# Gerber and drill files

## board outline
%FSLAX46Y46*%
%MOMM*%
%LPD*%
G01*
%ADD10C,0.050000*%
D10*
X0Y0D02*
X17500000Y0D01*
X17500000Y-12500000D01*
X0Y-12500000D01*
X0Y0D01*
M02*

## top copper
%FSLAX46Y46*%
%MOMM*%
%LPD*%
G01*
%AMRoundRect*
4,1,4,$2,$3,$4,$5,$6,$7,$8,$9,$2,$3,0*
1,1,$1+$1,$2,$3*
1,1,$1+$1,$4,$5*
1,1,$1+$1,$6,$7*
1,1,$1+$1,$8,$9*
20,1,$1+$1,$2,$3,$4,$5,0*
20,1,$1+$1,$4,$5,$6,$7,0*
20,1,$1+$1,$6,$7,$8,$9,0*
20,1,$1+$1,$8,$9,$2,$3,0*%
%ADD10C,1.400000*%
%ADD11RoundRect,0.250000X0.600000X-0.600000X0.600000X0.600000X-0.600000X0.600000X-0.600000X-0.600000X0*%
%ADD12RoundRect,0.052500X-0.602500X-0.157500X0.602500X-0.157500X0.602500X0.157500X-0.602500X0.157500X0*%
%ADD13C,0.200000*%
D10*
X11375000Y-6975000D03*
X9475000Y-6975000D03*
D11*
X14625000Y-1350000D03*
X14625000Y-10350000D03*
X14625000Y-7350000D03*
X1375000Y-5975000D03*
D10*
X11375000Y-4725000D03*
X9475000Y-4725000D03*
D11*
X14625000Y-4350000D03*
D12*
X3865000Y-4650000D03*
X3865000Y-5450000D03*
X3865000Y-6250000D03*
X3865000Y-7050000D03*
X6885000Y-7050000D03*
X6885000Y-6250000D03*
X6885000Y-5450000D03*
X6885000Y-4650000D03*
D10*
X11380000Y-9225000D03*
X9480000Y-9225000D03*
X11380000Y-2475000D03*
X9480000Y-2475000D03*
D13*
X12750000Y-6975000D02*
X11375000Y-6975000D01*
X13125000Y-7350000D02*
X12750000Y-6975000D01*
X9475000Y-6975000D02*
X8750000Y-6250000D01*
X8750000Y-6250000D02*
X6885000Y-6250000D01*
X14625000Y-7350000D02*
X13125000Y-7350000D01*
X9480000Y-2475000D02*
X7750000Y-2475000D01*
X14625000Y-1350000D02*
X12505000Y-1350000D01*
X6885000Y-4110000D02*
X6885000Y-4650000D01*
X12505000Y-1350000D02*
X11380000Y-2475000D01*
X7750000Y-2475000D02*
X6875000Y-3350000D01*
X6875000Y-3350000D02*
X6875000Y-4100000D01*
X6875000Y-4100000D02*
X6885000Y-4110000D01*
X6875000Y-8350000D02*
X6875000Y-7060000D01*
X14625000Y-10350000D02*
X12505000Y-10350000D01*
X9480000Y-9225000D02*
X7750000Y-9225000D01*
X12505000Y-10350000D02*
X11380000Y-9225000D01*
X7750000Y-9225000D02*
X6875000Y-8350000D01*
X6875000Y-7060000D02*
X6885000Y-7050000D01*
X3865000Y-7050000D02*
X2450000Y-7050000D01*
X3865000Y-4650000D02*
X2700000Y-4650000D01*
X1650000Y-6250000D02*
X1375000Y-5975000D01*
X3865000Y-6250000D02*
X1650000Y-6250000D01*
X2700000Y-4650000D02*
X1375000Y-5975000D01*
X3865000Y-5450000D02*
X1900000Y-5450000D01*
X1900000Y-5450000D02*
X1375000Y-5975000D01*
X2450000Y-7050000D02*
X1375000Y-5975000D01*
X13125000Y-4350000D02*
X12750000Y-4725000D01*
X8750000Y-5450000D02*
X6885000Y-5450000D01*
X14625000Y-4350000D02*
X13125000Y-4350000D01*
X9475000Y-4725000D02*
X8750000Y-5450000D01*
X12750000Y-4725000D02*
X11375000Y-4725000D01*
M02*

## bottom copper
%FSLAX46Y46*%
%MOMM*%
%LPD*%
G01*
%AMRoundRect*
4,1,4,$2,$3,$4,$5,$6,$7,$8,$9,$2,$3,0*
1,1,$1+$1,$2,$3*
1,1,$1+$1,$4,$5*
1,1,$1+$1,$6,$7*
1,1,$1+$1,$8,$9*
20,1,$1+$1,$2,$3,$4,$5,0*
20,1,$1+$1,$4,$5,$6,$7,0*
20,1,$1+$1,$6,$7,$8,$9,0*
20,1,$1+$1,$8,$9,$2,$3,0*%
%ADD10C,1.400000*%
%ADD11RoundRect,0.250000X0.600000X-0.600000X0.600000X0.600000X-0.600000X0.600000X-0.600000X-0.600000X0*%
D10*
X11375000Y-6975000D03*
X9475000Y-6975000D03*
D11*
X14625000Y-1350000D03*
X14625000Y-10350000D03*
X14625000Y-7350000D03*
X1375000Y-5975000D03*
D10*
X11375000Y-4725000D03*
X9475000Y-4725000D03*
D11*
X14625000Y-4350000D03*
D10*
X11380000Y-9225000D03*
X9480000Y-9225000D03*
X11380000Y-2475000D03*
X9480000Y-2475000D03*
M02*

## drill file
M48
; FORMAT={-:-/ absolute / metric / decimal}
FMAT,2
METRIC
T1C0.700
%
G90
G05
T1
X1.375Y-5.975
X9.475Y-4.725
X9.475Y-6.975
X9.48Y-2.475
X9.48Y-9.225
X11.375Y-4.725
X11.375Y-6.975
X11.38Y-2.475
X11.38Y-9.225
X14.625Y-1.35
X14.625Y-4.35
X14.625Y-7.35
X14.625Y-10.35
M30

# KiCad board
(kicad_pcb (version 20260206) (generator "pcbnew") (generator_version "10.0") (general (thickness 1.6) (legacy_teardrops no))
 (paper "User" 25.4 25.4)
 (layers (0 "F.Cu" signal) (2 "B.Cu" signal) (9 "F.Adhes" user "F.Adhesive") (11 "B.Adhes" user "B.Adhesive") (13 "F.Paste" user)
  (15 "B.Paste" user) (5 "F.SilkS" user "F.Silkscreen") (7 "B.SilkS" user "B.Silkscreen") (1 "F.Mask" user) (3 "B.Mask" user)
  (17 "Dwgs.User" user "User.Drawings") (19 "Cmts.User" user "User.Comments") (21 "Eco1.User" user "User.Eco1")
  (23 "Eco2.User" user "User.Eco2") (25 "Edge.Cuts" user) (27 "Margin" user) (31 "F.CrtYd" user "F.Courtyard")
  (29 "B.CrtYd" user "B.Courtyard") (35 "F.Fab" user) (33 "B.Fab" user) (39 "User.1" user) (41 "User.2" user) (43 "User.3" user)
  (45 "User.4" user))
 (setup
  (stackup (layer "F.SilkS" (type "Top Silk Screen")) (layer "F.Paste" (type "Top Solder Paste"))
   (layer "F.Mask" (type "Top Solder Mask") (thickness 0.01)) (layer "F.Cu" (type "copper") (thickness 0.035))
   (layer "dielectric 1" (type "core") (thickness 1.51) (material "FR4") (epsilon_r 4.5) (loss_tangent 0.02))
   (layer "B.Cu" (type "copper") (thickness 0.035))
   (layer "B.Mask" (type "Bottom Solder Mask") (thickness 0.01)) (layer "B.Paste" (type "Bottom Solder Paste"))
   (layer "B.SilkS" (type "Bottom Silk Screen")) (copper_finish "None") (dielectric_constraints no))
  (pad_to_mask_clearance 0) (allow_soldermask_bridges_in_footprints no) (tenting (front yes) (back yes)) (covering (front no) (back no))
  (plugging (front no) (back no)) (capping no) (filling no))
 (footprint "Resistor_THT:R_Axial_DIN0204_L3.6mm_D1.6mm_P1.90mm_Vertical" (layer "F.Cu") (at 11.375 6.975 180)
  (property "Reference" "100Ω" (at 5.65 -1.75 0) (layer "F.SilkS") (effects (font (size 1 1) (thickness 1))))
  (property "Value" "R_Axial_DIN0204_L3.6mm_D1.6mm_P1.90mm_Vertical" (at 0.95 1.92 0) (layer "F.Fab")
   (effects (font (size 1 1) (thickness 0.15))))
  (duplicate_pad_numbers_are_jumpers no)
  (pad "1" thru_hole circle (at 0 0 180) (size 1.4 1.4) (drill 0.7) (layers "*.Cu" "*.Mask") (remove_unused_layers no) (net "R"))
  (pad "2" thru_hole circle (at 1.9 0 180) (size 1.4 1.4) (drill 0.7) (layers "*.Cu" "*.Mask") (remove_unused_layers no) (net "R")))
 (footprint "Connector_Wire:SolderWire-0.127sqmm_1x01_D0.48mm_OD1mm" (layer "F.Cu") (at 14.625 1.35 90)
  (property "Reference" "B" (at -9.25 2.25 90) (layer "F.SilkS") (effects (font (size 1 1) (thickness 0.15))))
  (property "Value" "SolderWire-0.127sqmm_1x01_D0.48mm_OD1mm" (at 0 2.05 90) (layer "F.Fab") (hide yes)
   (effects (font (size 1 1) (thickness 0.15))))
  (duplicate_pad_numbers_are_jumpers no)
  (pad "1" thru_hole roundrect (at 0 0 90) (size 1.7 1.7) (drill 0.7) (layers "*.Cu" "*.Mask") (remove_unused_layers no)
   (roundrect_rratio 0.147059) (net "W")))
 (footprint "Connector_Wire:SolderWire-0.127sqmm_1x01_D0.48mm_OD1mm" (layer "F.Cu") (at 14.625 10.35 90)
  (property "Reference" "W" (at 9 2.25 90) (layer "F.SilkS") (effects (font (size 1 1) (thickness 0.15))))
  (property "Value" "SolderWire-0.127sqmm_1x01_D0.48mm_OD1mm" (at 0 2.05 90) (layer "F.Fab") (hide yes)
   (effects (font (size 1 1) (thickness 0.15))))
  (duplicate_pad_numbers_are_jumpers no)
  (pad "1" thru_hole roundrect (at 0 0 90) (size 1.7 1.7) (drill 0.7) (layers "*.Cu" "*.Mask") (remove_unused_layers no)
   (roundrect_rratio 0.147059) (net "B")))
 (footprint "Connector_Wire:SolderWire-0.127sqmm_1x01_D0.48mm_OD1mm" (layer "F.Cu") (at 14.625 7.35 90)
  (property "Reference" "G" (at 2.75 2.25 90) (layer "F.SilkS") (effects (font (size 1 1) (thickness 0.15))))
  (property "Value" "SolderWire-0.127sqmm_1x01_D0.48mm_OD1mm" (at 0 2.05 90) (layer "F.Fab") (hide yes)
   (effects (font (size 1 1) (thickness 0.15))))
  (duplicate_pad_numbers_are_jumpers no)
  (pad "1" thru_hole roundrect (at 0 0 90) (size 1.7 1.7) (drill 0.7) (layers "*.Cu" "*.Mask") (remove_unused_layers no)
   (roundrect_rratio 0.147059) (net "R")))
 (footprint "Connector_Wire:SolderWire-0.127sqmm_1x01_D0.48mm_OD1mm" (layer "F.Cu") (at 1.375 5.975 90)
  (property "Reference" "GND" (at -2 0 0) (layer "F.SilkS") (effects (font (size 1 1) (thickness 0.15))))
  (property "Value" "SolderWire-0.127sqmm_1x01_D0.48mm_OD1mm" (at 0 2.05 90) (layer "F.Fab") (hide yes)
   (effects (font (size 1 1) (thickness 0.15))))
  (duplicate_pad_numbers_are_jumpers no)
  (pad "1" thru_hole roundrect (at 0 0 90) (size 1.7 1.7) (drill 0.7) (layers "*.Cu" "*.Mask") (remove_unused_layers no)
   (roundrect_rratio 0.147059) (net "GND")))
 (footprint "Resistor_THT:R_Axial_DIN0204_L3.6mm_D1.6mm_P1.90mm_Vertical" (layer "F.Cu") (at 11.375 4.725 180)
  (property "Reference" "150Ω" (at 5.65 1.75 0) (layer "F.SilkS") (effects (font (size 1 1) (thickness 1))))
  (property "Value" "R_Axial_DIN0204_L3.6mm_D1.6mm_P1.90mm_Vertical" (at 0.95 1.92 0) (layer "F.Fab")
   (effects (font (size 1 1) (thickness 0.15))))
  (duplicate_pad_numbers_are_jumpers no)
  (pad "1" thru_hole circle (at 0 0 180) (size 1.4 1.4) (drill 0.7) (layers "*.Cu" "*.Mask") (remove_unused_layers no) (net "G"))
  (pad "2" thru_hole circle (at 1.9 0 180) (size 1.4 1.4) (drill 0.7) (layers "*.Cu" "*.Mask") (remove_unused_layers no) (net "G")))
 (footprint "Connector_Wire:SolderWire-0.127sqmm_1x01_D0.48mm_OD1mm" (layer "F.Cu") (at 14.625 4.35 90)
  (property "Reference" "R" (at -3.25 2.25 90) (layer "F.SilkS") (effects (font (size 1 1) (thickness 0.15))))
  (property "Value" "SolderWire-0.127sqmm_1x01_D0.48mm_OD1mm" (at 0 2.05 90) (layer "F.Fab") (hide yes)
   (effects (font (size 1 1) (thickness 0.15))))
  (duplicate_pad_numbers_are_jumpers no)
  (pad "1" thru_hole roundrect (at 0 0 90) (size 1.7 1.7) (drill 0.7) (layers "*.Cu" "*.Mask") (remove_unused_layers no)
   (roundrect_rratio 0.147059) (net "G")))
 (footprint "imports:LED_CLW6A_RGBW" (layer "F.Cu") (at 5.375 5.85)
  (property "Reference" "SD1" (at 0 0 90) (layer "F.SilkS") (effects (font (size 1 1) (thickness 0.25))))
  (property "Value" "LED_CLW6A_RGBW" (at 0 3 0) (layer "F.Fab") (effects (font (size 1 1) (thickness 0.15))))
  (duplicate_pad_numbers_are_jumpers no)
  (pad "1" smd roundrect (at -1.51 -1.2) (size 1.31 0.42) (layers "F.Cu" "F.Mask" "F.Paste") (roundrect_rratio 0.125) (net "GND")
   (solder_mask_margin 0.102))
  (pad "2" smd roundrect (at -1.51 -0.4) (size 1.31 0.42) (layers "F.Cu" "F.Mask" "F.Paste") (roundrect_rratio 0.125) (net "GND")
   (solder_mask_margin 0.102))
  (pad "3" smd roundrect (at -1.51 0.4) (size 1.31 0.42) (layers "F.Cu" "F.Mask" "F.Paste") (roundrect_rratio 0.125) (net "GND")
   (solder_mask_margin 0.102))
  (pad "4" smd roundrect (at -1.51 1.2) (size 1.31 0.42) (layers "F.Cu" "F.Mask" "F.Paste") (roundrect_rratio 0.125) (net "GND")
   (solder_mask_margin 0.102))
  (pad "5" smd roundrect (at 1.51 1.2) (size 1.31 0.42) (layers "F.Cu" "F.Mask" "F.Paste") (roundrect_rratio 0.125) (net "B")
   (solder_mask_margin 0.102))
  (pad "6" smd roundrect (at 1.51 0.4) (size 1.31 0.42) (layers "F.Cu" "F.Mask" "F.Paste") (roundrect_rratio 0.125) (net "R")
   (solder_mask_margin 0.102))
  (pad "7" smd roundrect (at 1.51 -0.4) (size 1.31 0.42) (layers "F.Cu" "F.Mask" "F.Paste") (roundrect_rratio 0.125) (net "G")
   (solder_mask_margin 0.102))
  (pad "8" smd roundrect (at 1.51 -1.2) (size 1.31 0.42) (layers "F.Cu" "F.Mask" "F.Paste") (roundrect_rratio 0.125) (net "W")
   (solder_mask_margin 0.102)))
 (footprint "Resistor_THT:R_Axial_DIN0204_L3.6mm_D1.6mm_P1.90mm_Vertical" (layer "F.Cu") (at 11.38 9.225 180)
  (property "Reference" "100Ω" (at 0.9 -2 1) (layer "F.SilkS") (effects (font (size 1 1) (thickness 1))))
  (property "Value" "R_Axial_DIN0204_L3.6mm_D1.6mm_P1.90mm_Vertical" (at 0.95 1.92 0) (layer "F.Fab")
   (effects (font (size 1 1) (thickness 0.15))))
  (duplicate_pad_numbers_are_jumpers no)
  (pad "1" thru_hole circle (at 0 0 180) (size 1.4 1.4) (drill 0.7) (layers "*.Cu" "*.Mask") (remove_unused_layers no) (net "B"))
  (pad "2" thru_hole circle (at 1.9 0 180) (size 1.4 1.4) (drill 0.7) (layers "*.Cu" "*.Mask") (remove_unused_layers no) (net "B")))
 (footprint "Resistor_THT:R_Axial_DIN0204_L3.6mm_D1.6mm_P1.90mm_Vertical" (layer "F.Cu") (at 11.38 2.475 180)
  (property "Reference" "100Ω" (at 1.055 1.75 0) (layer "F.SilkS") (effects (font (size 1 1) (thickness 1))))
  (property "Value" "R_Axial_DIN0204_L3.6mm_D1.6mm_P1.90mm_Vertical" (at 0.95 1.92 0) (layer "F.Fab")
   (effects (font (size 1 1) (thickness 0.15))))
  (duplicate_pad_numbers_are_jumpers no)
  (pad "1" thru_hole circle (at 0 0 180) (size 1.4 1.4) (drill 0.7) (layers "*.Cu" "*.Mask") (remove_unused_layers no) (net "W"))
  (pad "2" thru_hole circle (at 1.9 0 180) (size 1.4 1.4) (drill 0.7) (layers "*.Cu" "*.Mask") (remove_unused_layers no) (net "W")))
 (gr_rect (start 0 0) (end 17.5 12.5) (stroke (width 0.05) (type default)) (fill no) (layer "Edge.Cuts"))
 (segment (start 12.75 6.975) (end 11.375 6.975) (width 0.2) (layer "F.Cu") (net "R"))
 (segment (start 13.125 7.35) (end 12.75 6.975) (width 0.2) (layer "F.Cu") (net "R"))
 (segment (start 9.475 6.975) (end 8.75 6.25) (width 0.2) (layer "F.Cu") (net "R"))
 (segment (start 8.75 6.25) (end 6.885 6.25) (width 0.2) (layer "F.Cu") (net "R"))
 (segment (start 14.625 7.35) (end 13.125 7.35) (width 0.2) (layer "F.Cu") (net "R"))
 (segment (start 9.48 2.475) (end 7.75 2.475) (width 0.2) (layer "F.Cu") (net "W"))
 (segment (start 14.625 1.35) (end 12.505 1.35) (width 0.2) (layer "F.Cu") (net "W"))
 (segment (start 6.885 4.11) (end 6.885 4.65) (width 0.2) (layer "F.Cu") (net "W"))
 (segment (start 12.505 1.35) (end 11.38 2.475) (width 0.2) (layer "F.Cu") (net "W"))
 (segment (start 7.75 2.475) (end 6.875 3.35) (width 0.2) (layer "F.Cu") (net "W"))
 (segment (start 6.875 3.35) (end 6.875 4.1) (width 0.2) (layer "F.Cu") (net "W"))
 (segment (start 6.875 4.1) (end 6.885 4.11) (width 0.2) (layer "F.Cu") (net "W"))
 (segment (start 6.875 8.35) (end 6.875 7.06) (width 0.2) (layer "F.Cu") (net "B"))
 (segment (start 14.625 10.35) (end 12.505 10.35) (width 0.2) (layer "F.Cu") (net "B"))
 (segment (start 9.48 9.225) (end 7.75 9.225) (width 0.2) (layer "F.Cu") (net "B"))
 (segment (start 12.505 10.35) (end 11.38 9.225) (width 0.2) (layer "F.Cu") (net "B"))
 (segment (start 7.75 9.225) (end 6.875 8.35) (width 0.2) (layer "F.Cu") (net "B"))
 (segment (start 6.875 7.06) (end 6.885 7.05) (width 0.2) (layer "F.Cu") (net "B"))
 (segment (start 3.865 7.05) (end 2.45 7.05) (width 0.2) (layer "F.Cu") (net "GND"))
 (segment (start 3.865 4.65) (end 2.7 4.65) (width 0.2) (layer "F.Cu") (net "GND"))
 (segment (start 1.65 6.25) (end 1.375 5.975) (width 0.2) (layer "F.Cu") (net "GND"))
 (segment (start 3.865 6.25) (end 1.65 6.25) (width 0.2) (layer "F.Cu") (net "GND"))
 (segment (start 2.7 4.65) (end 1.375 5.975) (width 0.2) (layer "F.Cu") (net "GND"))
 (segment (start 3.865 5.45) (end 1.9 5.45) (width 0.2) (layer "F.Cu") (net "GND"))
 (segment (start 1.9 5.45) (end 1.375 5.975) (width 0.2) (layer "F.Cu") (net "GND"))
 (segment (start 2.45 7.05) (end 1.375 5.975) (width 0.2) (layer "F.Cu") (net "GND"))
 (segment (start 13.125 4.35) (end 12.75 4.725) (width 0.2) (layer "F.Cu") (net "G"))
 (segment (start 8.75 5.45) (end 6.885 5.45) (width 0.2) (layer "F.Cu") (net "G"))
 (segment (start 14.625 4.35) (end 13.125 4.35) (width 0.2) (layer "F.Cu") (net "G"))
 (segment (start 9.475 4.725) (end 8.75 5.45) (width 0.2) (layer "F.Cu") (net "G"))
 (segment (start 12.75 4.725) (end 11.375 4.725) (width 0.2) (layer "F.Cu") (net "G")))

